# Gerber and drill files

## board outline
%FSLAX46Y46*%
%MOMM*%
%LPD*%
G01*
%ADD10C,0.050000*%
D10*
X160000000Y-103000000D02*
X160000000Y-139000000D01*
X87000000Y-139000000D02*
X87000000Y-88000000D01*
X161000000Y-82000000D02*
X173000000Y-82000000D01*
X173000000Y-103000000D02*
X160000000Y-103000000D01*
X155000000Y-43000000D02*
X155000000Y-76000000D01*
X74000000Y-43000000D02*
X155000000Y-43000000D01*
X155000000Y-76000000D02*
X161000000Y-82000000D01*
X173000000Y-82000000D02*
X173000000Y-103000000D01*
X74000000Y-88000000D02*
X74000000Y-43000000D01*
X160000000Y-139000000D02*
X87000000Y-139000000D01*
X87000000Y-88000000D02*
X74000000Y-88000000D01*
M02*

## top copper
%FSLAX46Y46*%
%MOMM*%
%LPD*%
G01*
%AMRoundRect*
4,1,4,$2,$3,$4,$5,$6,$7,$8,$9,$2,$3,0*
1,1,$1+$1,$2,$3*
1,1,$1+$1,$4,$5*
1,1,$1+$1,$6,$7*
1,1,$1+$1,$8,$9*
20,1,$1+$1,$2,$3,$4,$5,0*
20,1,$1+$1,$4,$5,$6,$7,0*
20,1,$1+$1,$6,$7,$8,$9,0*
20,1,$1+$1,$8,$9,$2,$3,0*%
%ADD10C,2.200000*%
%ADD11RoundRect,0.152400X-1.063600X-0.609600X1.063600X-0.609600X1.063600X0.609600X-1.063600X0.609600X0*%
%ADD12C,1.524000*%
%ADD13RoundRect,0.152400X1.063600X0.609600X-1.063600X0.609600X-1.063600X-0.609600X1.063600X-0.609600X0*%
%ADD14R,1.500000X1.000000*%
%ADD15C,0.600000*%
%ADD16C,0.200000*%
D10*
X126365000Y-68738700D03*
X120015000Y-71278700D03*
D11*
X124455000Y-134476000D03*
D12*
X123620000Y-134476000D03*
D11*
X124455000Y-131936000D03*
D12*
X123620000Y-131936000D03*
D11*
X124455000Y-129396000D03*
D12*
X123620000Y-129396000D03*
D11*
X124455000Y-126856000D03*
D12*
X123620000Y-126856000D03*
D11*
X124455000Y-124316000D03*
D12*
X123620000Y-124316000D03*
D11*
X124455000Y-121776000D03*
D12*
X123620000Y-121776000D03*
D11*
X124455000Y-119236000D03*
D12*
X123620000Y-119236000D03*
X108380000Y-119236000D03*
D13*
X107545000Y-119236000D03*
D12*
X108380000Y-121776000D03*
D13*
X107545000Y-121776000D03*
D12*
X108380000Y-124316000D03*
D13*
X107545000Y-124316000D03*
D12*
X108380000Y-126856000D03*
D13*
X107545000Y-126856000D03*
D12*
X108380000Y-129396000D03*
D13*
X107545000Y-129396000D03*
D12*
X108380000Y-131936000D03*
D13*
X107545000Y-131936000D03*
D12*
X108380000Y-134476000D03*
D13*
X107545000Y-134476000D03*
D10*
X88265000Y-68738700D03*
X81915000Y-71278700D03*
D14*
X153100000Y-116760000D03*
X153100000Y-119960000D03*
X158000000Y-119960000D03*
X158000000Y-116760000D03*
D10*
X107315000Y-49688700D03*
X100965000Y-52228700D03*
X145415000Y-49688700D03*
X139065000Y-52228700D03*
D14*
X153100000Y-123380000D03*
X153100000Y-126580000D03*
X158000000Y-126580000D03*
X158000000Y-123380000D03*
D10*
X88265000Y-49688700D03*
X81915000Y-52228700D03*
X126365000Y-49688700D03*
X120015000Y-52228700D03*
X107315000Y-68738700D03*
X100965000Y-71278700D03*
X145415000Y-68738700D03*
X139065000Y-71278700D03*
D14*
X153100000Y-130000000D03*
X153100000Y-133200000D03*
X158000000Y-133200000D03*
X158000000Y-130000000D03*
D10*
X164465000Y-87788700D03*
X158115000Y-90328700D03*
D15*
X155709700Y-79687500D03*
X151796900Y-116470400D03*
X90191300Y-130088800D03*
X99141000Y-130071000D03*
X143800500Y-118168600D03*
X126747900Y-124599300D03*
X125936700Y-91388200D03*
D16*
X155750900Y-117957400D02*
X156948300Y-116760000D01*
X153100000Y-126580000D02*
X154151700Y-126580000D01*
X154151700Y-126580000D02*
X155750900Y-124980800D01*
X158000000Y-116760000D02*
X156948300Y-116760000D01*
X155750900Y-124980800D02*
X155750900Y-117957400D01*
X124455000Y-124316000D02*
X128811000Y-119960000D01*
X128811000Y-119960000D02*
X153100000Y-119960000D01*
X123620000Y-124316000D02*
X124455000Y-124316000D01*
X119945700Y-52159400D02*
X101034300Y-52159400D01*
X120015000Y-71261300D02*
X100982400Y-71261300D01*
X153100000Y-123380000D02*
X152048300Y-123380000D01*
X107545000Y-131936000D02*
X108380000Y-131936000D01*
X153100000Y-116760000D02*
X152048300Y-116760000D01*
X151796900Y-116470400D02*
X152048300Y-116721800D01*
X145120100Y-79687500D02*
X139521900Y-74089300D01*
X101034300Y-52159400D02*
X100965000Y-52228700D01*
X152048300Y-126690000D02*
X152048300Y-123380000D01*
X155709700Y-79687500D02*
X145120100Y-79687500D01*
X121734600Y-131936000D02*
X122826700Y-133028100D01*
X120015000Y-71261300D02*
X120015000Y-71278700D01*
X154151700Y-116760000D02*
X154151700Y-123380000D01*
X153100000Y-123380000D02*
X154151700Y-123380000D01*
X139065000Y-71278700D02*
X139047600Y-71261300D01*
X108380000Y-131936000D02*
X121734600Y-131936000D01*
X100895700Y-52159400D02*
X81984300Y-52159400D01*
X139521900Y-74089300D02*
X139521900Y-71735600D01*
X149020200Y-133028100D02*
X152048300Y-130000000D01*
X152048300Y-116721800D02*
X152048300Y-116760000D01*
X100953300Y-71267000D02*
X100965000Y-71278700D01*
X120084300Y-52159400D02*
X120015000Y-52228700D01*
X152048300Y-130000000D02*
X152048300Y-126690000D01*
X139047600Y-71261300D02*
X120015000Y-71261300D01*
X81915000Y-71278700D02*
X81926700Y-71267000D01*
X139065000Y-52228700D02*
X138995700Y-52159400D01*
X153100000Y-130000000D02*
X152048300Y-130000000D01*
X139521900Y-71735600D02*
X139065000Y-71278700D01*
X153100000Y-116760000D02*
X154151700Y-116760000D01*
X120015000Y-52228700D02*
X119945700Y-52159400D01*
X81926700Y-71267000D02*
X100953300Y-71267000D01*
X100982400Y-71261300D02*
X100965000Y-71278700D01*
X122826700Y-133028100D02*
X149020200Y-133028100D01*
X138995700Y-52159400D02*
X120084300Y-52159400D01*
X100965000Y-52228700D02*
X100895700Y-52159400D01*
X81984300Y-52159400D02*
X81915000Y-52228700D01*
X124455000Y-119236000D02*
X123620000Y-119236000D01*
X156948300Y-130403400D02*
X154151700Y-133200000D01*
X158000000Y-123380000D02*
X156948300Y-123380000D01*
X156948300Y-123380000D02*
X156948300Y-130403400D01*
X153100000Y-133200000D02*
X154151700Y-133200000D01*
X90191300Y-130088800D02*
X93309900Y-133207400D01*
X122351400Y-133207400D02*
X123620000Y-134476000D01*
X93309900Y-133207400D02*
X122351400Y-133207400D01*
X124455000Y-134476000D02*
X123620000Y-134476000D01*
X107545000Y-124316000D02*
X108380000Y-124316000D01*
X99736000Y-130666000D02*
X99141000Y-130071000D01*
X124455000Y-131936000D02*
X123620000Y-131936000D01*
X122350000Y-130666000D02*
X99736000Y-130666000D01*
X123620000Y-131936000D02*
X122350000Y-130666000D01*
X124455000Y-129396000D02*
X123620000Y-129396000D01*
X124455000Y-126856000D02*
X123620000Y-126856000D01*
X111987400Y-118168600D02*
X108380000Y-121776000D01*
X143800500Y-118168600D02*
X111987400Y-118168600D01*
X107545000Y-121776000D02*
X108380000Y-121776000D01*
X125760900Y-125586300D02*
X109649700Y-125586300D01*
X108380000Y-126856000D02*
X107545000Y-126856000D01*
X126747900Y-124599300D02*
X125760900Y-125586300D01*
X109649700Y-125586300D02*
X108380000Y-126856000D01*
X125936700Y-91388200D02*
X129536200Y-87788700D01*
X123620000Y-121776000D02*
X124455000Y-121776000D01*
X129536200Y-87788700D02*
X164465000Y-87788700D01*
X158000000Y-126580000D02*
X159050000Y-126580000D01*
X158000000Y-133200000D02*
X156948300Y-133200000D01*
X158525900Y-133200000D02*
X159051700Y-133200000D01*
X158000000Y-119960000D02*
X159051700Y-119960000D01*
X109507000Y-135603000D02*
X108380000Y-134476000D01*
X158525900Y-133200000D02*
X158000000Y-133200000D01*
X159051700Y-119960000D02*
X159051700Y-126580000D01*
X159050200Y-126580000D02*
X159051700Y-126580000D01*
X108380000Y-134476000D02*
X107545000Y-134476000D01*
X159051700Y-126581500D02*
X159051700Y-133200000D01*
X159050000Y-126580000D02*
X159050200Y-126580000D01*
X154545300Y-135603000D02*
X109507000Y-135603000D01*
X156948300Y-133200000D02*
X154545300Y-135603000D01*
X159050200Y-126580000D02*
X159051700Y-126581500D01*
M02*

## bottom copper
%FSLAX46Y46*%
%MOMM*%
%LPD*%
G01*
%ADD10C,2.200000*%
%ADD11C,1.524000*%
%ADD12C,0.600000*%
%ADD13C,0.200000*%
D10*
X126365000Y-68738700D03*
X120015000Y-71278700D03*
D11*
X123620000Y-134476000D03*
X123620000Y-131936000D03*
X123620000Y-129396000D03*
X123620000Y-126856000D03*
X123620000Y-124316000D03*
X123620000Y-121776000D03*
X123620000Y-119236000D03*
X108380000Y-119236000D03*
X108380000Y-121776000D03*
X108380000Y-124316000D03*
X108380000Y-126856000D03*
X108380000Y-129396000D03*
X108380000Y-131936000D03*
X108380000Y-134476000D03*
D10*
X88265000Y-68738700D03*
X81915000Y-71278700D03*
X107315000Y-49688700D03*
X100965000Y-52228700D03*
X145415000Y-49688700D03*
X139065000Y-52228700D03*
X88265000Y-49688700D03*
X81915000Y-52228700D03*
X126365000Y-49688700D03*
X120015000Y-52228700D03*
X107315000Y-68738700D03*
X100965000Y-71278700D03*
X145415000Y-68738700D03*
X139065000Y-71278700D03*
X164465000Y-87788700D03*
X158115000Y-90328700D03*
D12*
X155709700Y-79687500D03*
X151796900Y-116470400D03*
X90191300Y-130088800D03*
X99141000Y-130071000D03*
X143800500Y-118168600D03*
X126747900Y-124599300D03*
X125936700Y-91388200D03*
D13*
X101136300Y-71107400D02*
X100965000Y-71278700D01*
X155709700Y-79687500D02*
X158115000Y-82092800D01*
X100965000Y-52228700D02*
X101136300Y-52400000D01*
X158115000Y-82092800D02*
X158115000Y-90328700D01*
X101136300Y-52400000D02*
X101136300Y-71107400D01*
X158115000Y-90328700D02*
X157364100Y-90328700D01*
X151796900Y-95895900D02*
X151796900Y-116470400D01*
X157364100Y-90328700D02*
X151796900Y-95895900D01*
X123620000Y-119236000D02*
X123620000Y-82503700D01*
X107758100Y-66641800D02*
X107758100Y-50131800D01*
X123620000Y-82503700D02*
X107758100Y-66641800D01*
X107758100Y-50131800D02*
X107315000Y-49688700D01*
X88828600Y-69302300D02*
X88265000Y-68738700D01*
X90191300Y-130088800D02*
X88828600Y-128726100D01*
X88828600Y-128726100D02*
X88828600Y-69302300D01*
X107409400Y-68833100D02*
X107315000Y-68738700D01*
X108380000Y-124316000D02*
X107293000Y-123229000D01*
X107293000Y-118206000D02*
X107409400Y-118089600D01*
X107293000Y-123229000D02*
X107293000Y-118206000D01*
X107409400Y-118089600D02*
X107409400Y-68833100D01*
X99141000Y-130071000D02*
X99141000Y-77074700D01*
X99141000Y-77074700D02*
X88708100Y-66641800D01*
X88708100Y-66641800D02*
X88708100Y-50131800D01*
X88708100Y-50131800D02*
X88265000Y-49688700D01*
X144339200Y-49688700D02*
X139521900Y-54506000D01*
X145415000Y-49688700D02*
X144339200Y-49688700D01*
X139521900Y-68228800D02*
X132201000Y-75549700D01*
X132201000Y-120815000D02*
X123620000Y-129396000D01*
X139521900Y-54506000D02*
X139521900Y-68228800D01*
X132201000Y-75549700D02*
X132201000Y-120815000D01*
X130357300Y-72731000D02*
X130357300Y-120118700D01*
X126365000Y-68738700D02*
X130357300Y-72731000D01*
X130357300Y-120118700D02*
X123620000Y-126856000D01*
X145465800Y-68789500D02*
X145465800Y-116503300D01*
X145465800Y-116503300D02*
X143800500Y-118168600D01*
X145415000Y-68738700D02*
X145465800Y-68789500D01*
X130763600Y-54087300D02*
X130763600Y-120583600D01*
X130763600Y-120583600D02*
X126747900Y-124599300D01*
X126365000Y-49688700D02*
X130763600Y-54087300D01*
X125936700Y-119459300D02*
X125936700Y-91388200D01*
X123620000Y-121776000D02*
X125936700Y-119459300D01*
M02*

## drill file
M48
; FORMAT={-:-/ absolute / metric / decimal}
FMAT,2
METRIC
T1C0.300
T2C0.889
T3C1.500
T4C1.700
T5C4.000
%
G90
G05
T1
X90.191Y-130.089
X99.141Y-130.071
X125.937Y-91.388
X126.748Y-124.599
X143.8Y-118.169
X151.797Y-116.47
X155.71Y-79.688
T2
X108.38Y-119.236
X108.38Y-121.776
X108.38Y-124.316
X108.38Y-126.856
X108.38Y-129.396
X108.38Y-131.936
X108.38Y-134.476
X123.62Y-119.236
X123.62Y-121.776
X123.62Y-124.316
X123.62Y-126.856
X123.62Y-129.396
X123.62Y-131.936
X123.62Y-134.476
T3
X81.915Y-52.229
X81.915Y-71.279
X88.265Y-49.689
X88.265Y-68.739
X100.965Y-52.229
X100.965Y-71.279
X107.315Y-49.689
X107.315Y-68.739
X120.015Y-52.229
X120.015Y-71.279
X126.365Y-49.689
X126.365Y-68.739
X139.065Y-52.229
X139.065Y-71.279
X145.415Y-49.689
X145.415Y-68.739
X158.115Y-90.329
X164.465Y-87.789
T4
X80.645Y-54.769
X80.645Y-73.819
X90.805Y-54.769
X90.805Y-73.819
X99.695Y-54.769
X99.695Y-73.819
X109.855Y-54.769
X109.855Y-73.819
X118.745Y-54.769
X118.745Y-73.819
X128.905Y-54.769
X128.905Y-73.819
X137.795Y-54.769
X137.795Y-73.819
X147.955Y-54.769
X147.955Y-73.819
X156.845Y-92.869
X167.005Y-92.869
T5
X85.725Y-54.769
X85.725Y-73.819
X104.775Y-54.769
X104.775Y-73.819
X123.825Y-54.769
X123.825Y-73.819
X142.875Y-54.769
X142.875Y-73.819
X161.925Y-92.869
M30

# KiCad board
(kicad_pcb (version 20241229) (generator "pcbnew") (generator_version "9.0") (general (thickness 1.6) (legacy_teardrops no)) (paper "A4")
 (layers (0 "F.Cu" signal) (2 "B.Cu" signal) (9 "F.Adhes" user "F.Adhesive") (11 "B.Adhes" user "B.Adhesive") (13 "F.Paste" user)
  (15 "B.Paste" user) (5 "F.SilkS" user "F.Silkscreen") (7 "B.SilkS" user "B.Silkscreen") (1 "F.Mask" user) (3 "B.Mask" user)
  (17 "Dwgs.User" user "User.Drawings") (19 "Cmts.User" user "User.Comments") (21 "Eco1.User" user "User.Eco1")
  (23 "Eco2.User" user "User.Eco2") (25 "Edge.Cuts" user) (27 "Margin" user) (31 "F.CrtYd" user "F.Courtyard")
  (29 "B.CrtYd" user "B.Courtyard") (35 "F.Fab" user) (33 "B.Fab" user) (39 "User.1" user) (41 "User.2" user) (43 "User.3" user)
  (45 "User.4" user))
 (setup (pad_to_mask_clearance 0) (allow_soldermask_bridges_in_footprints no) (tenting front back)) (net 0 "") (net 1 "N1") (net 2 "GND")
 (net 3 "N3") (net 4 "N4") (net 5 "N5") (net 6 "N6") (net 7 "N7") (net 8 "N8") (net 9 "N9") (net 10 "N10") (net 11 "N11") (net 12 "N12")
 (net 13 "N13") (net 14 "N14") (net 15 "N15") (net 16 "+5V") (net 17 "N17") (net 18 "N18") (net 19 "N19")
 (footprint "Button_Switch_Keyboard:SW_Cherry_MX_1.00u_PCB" (layer "F.Cu") (at 126.365 68.7387)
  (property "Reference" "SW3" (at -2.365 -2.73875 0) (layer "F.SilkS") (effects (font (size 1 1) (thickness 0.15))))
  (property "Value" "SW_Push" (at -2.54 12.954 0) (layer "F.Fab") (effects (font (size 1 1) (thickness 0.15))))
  (pad "" np_thru_hole circle (at -7.62 5.08) (size 1.7 1.7) (drill 1.7) (layers "*.Cu" "*.Mask"))
  (pad "" np_thru_hole circle (at -2.54 5.08) (size 4 4) (drill 4) (layers "*.Cu" "*.Mask"))
  (pad "" np_thru_hole circle (at 2.54 5.08) (size 1.7 1.7) (drill 1.7) (layers "*.Cu" "*.Mask"))
  (pad "1" thru_hole circle (at 0 0) (size 2.2 2.2) (drill 1.5) (layers "*.Cu" "*.Mask") (remove_unused_layers no) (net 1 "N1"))
  (pad "2" thru_hole circle (at -6.35 2.54) (size 2.2 2.2) (drill 1.5) (layers "*.Cu" "*.Mask") (remove_unused_layers no) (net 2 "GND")))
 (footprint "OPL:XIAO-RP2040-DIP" (layer "F.Cu") (at 116 126.856 180)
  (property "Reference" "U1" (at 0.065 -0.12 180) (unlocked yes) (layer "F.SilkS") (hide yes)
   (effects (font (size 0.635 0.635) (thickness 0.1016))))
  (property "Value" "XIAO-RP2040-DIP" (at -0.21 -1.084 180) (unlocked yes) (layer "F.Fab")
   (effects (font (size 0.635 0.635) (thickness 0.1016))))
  (pad "1" smd roundrect (at -8.455 -7.62) (size 2.432 1.524) (layers "F.Cu" "F.Mask") (roundrect_rratio 0.1) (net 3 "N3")
   (thermal_bridge_angle 45))
  (pad "1" thru_hole circle (at -7.62 -7.62) (size 1.524 1.524) (drill 0.889) (layers "*.Cu" "*.Mask") (remove_unused_layers no)
   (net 3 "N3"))
  (pad "2" smd roundrect (at -8.455 -5.08) (size 2.432 1.524) (layers "F.Cu" "F.Mask") (roundrect_rratio 0.1) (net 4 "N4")
   (thermal_bridge_angle 45))
  (pad "2" thru_hole circle (at -7.62 -5.08) (size 1.524 1.524) (drill 0.889) (layers "*.Cu" "*.Mask") (remove_unused_layers no)
   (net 4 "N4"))
  (pad "3" smd roundrect (at -8.455 -2.54) (size 2.432 1.524) (layers "F.Cu" "F.Mask") (roundrect_rratio 0.1) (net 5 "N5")
   (thermal_bridge_angle 45))
  (pad "3" thru_hole circle (at -7.62 -2.54) (size 1.524 1.524) (drill 0.889) (layers "*.Cu" "*.Mask") (remove_unused_layers no)
   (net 5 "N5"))
  (pad "4" smd roundrect (at -8.455 0) (size 2.432 1.524) (layers "F.Cu" "F.Mask") (roundrect_rratio 0.1) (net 1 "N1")
   (thermal_bridge_angle 45))
  (pad "4" thru_hole circle (at -7.62 0) (size 1.524 1.524) (drill 0.889) (layers "*.Cu" "*.Mask") (remove_unused_layers no) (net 1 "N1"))
  (pad "5" smd roundrect (at -8.455 2.54) (size 2.432 1.524) (layers "F.Cu" "F.Mask") (roundrect_rratio 0.1) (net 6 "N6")
   (thermal_bridge_angle 45))
  (pad "5" thru_hole circle (at -7.62 2.54) (size 1.524 1.524) (drill 0.889) (layers "*.Cu" "*.Mask") (remove_unused_layers no) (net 6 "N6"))
  (pad "6" smd roundrect (at -8.455 5.08) (size 2.432 1.524) (layers "F.Cu" "F.Mask") (roundrect_rratio 0.1) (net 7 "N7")
   (thermal_bridge_angle 45))
  (pad "6" thru_hole circle (at -7.62 5.08) (size 1.524 1.524) (drill 0.889) (layers "*.Cu" "*.Mask") (remove_unused_layers no) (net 7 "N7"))
  (pad "7" smd roundrect (at -8.455 7.62) (size 2.432 1.524) (layers "F.Cu" "F.Mask") (roundrect_rratio 0.1) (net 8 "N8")
   (thermal_bridge_angle 45))
  (pad "7" thru_hole circle (at -7.62 7.62) (size 1.524 1.524) (drill 0.889) (layers "*.Cu" "*.Mask") (remove_unused_layers no) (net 8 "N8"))
  (pad "8" thru_hole circle (at 7.62 7.62 180) (size 1.524 1.524) (drill 0.889) (layers "*.Cu" "*.Mask") (remove_unused_layers no)
   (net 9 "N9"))
  (pad "8" smd roundrect (at 8.455 7.62 180) (size 2.432 1.524) (layers "F.Cu" "F.Mask") (roundrect_rratio 0.1) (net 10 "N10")
   (thermal_bridge_angle 45))
  (pad "9" thru_hole circle (at 7.62 5.08 180) (size 1.524 1.524) (drill 0.889) (layers "*.Cu" "*.Mask") (remove_unused_layers no)
   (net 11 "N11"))
  (pad "9" smd roundrect (at 8.455 5.08 180) (size 2.432 1.524) (layers "F.Cu" "F.Mask") (roundrect_rratio 0.1) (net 11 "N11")
   (thermal_bridge_angle 45))
  (pad "10" thru_hole circle (at 7.62 2.54 180) (size 1.524 1.524) (drill 0.889) (layers "*.Cu" "*.Mask") (remove_unused_layers no)
   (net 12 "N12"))
  (pad "10" smd roundrect (at 8.455 2.54 180) (size 2.432 1.524) (layers "F.Cu" "F.Mask") (roundrect_rratio 0.1) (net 12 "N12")
   (thermal_bridge_angle 45))
  (pad "11" thru_hole circle (at 7.62 0 180) (size 1.524 1.524) (drill 0.889) (layers "*.Cu" "*.Mask") (remove_unused_layers no)
   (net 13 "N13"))
  (pad "11" smd roundrect (at 8.455 0 180) (size 2.432 1.524) (layers "F.Cu" "F.Mask") (roundrect_rratio 0.1) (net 13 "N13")
   (thermal_bridge_angle 45))
  (pad "12" thru_hole circle (at 7.62 -2.54 180) (size 1.524 1.524) (drill 0.889) (layers "*.Cu" "*.Mask") (remove_unused_layers no)
   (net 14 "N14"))
  (pad "12" smd roundrect (at 8.455 -2.54 180) (size 2.432 1.524) (layers "F.Cu" "F.Mask") (roundrect_rratio 0.1) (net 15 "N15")
   (thermal_bridge_angle 45))
  (pad "13" thru_hole circle (at 7.62 -5.08 180) (size 1.524 1.524) (drill 0.889) (layers "*.Cu" "*.Mask") (remove_unused_layers no)
   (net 2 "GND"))
  (pad "13" smd roundrect (at 8.455 -5.08 180) (size 2.432 1.524) (layers "F.Cu" "F.Mask") (roundrect_rratio 0.1) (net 2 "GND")
   (thermal_bridge_angle 45))
  (pad "14" thru_hole circle (at 7.62 -7.62 180) (size 1.524 1.524) (drill 0.889) (layers "*.Cu" "*.Mask") (remove_unused_layers no)
   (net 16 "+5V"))
  (pad "14" smd roundrect (at 8.455 -7.62 180) (size 2.432 1.524) (layers "F.Cu" "F.Mask") (roundrect_rratio 0.1) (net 16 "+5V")
   (thermal_bridge_angle 45)))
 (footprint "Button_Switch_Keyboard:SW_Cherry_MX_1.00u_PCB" (layer "F.Cu") (at 88.265 68.7387)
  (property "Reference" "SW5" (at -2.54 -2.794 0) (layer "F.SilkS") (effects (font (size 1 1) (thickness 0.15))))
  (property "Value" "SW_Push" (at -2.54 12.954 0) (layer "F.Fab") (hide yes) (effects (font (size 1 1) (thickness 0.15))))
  (pad "" np_thru_hole circle (at -7.62 5.08) (size 1.7 1.7) (drill 1.7) (layers "*.Cu" "*.Mask"))
  (pad "" np_thru_hole circle (at -2.54 5.08) (size 4 4) (drill 4) (layers "*.Cu" "*.Mask"))
  (pad "" np_thru_hole circle (at 2.54 5.08) (size 1.7 1.7) (drill 1.7) (layers "*.Cu" "*.Mask"))
  (pad "1" thru_hole circle (at 0 0) (size 2.2 2.2) (drill 1.5) (layers "*.Cu" "*.Mask") (remove_unused_layers no) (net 3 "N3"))
  (pad "2" thru_hole circle (at -6.35 2.54) (size 2.2 2.2) (drill 1.5) (layers "*.Cu" "*.Mask") (remove_unused_layers no) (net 2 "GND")))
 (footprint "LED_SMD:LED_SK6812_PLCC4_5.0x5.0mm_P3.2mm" (layer "F.Cu") (at 155.55 118.36)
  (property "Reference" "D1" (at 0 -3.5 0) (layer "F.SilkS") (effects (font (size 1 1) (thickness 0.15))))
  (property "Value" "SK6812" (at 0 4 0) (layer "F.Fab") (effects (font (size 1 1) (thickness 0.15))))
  (pad "1" smd rect (at -2.45 -1.6 180) (size 1.5 1) (layers "F.Cu" "F.Mask" "F.Paste") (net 2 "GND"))
  (pad "2" smd rect (at -2.45 1.6 180) (size 1.5 1) (layers "F.Cu" "F.Mask" "F.Paste") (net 6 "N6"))
  (pad "3" smd rect (at 2.45 1.6 180) (size 1.5 1) (layers "F.Cu" "F.Mask" "F.Paste") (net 16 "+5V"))
  (pad "4" smd rect (at 2.45 -1.6 180) (size 1.5 1) (layers "F.Cu" "F.Mask" "F.Paste") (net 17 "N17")))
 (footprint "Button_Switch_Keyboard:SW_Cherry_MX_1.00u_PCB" (layer "F.Cu") (at 107.315 49.6887)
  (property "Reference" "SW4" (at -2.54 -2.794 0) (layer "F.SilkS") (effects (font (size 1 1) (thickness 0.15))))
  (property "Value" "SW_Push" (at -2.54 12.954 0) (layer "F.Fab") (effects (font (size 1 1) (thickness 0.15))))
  (pad "" np_thru_hole circle (at -7.62 5.08) (size 1.7 1.7) (drill 1.7) (layers "*.Cu" "*.Mask"))
  (pad "" np_thru_hole circle (at -2.54 5.08) (size 4 4) (drill 4) (layers "*.Cu" "*.Mask"))
  (pad "" np_thru_hole circle (at 2.54 5.08) (size 1.7 1.7) (drill 1.7) (layers "*.Cu" "*.Mask"))
  (pad "1" thru_hole circle (at 0 0) (size 2.2 2.2) (drill 1.5) (layers "*.Cu" "*.Mask") (remove_unused_layers no) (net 8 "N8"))
  (pad "2" thru_hole circle (at -6.35 2.54) (size 2.2 2.2) (drill 1.5) (layers "*.Cu" "*.Mask") (remove_unused_layers no) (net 2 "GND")))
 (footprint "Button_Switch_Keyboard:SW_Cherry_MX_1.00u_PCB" (layer "F.Cu") (at 145.415 49.6887)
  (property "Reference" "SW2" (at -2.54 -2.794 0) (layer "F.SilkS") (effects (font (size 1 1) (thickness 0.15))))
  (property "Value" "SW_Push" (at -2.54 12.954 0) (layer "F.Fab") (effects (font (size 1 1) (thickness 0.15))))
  (pad "" np_thru_hole circle (at -7.62 5.08) (size 1.7 1.7) (drill 1.7) (layers "*.Cu" "*.Mask"))
  (pad "" np_thru_hole circle (at -2.54 5.08) (size 4 4) (drill 4) (layers "*.Cu" "*.Mask"))
  (pad "" np_thru_hole circle (at 2.54 5.08) (size 1.7 1.7) (drill 1.7) (layers "*.Cu" "*.Mask"))
  (pad "1" thru_hole circle (at 0 0) (size 2.2 2.2) (drill 1.5) (layers "*.Cu" "*.Mask") (remove_unused_layers no) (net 5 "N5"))
  (pad "2" thru_hole circle (at -6.35 2.54) (size 2.2 2.2) (drill 1.5) (layers "*.Cu" "*.Mask") (remove_unused_layers no) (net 2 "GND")))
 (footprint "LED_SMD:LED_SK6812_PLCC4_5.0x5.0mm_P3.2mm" (layer "F.Cu") (at 155.55 124.98)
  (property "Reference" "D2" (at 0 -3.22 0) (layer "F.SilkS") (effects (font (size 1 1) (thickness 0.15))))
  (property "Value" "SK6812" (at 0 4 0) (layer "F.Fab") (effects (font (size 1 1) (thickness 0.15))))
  (pad "1" smd rect (at -2.45 -1.6 180) (size 1.5 1) (layers "F.Cu" "F.Mask" "F.Paste") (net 2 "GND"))
  (pad "2" smd rect (at -2.45 1.6 180) (size 1.5 1) (layers "F.Cu" "F.Mask" "F.Paste") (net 17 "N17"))
  (pad "3" smd rect (at 2.45 1.6 180) (size 1.5 1) (layers "F.Cu" "F.Mask" "F.Paste") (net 16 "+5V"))
  (pad "4" smd rect (at 2.45 -1.6 180) (size 1.5 1) (layers "F.Cu" "F.Mask" "F.Paste") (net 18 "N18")))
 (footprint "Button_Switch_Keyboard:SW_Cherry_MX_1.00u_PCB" (layer "F.Cu") (at 88.265 49.6887)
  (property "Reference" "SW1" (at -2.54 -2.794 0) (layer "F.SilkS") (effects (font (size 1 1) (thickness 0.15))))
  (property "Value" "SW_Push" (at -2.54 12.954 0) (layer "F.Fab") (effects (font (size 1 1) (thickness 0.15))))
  (pad "" np_thru_hole circle (at -7.62 5.08) (size 1.7 1.7) (drill 1.7) (layers "*.Cu" "*.Mask"))
  (pad "" np_thru_hole circle (at -2.54 5.08) (size 4 4) (drill 4) (layers "*.Cu" "*.Mask"))
  (pad "" np_thru_hole circle (at 2.54 5.08) (size 1.7 1.7) (drill 1.7) (layers "*.Cu" "*.Mask"))
  (pad "1" thru_hole circle (at 0 0) (size 2.2 2.2) (drill 1.5) (layers "*.Cu" "*.Mask") (remove_unused_layers no) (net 4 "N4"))
  (pad "2" thru_hole circle (at -6.35 2.54) (size 2.2 2.2) (drill 1.5) (layers "*.Cu" "*.Mask") (remove_unused_layers no) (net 2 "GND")))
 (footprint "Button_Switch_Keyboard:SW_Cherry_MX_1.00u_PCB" (layer "F.Cu") (at 126.365 49.6887)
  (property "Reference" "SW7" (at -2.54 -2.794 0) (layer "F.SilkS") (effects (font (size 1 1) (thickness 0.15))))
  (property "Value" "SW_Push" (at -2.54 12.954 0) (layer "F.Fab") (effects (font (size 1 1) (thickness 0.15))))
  (pad "" np_thru_hole circle (at -7.62 5.08) (size 1.7 1.7) (drill 1.7) (layers "*.Cu" "*.Mask"))
  (pad "" np_thru_hole circle (at -2.54 5.08) (size 4 4) (drill 4) (layers "*.Cu" "*.Mask"))
  (pad "" np_thru_hole circle (at 2.54 5.08) (size 1.7 1.7) (drill 1.7) (layers "*.Cu" "*.Mask"))
  (pad "1" thru_hole circle (at 0 0) (size 2.2 2.2) (drill 1.5) (layers "*.Cu" "*.Mask") (remove_unused_layers no) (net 13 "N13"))
  (pad "2" thru_hole circle (at -6.35 2.54) (size 2.2 2.2) (drill 1.5) (layers "*.Cu" "*.Mask") (remove_unused_layers no) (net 2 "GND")))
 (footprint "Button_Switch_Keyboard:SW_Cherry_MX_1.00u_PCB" (layer "F.Cu") (at 107.315 68.7387)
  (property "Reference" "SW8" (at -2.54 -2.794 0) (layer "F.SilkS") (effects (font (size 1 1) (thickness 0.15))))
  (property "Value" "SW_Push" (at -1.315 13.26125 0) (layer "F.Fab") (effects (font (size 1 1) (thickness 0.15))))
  (pad "" np_thru_hole circle (at -7.62 5.08) (size 1.7 1.7) (drill 1.7) (layers "*.Cu" "*.Mask"))
  (pad "" np_thru_hole circle (at -2.54 5.08) (size 4 4) (drill 4) (layers "*.Cu" "*.Mask"))
  (pad "" np_thru_hole circle (at 2.54 5.08) (size 1.7 1.7) (drill 1.7) (layers "*.Cu" "*.Mask"))
  (pad "1" thru_hole circle (at 0 0) (size 2.2 2.2) (drill 1.5) (layers "*.Cu" "*.Mask") (remove_unused_layers no) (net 12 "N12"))
  (pad "2" thru_hole circle (at -6.35 2.54) (size 2.2 2.2) (drill 1.5) (layers "*.Cu" "*.Mask") (remove_unused_layers no) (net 2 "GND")))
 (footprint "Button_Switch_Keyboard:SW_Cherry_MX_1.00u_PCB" (layer "F.Cu") (at 145.415 68.7387)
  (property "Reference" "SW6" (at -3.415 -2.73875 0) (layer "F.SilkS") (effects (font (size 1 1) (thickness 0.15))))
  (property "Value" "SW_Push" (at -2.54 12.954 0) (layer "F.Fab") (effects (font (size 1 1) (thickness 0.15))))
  (pad "" np_thru_hole circle (at -7.62 5.08) (size 1.7 1.7) (drill 1.7) (layers "*.Cu" "*.Mask"))
  (pad "" np_thru_hole circle (at -2.54 5.08) (size 4 4) (drill 4) (layers "*.Cu" "*.Mask"))
  (pad "" np_thru_hole circle (at 2.54 5.08) (size 1.7 1.7) (drill 1.7) (layers "*.Cu" "*.Mask"))
  (pad "1" thru_hole circle (at 0 0) (size 2.2 2.2) (drill 1.5) (layers "*.Cu" "*.Mask") (remove_unused_layers no) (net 11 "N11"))
  (pad "2" thru_hole circle (at -6.35 2.54) (size 2.2 2.2) (drill 1.5) (layers "*.Cu" "*.Mask") (remove_unused_layers no) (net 2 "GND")))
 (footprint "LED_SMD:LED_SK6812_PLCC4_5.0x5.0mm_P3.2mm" (layer "F.Cu") (at 155.55 131.6)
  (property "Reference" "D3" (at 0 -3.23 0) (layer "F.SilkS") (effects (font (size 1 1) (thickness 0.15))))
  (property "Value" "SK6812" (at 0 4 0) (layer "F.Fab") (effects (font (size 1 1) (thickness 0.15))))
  (pad "1" smd rect (at -2.45 -1.6 180) (size 1.5 1) (layers "F.Cu" "F.Mask" "F.Paste") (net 2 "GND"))
  (pad "2" smd rect (at -2.45 1.6 180) (size 1.5 1) (layers "F.Cu" "F.Mask" "F.Paste") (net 18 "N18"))
  (pad "3" smd rect (at 2.45 1.6 180) (size 1.5 1) (layers "F.Cu" "F.Mask" "F.Paste") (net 16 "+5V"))
  (pad "4" smd rect (at 2.45 -1.6 180) (size 1.5 1) (layers "F.Cu" "F.Mask" "F.Paste") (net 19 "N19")))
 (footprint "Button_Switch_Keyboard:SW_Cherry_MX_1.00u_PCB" (layer "F.Cu") (at 164.465 87.7887)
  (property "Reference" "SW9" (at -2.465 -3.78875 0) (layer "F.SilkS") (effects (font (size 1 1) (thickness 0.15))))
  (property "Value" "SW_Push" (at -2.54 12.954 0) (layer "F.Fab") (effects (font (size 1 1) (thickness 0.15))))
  (pad "" np_thru_hole circle (at -7.62 5.08) (size 1.7 1.7) (drill 1.7) (layers "*.Cu" "*.Mask"))
  (pad "" np_thru_hole circle (at -2.54 5.08) (size 4 4) (drill 4) (layers "*.Cu" "*.Mask"))
  (pad "" np_thru_hole circle (at 2.54 5.08) (size 1.7 1.7) (drill 1.7) (layers "*.Cu" "*.Mask"))
  (pad "1" thru_hole circle (at 0 0) (size 2.2 2.2) (drill 1.5) (layers "*.Cu" "*.Mask") (remove_unused_layers no) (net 7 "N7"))
  (pad "2" thru_hole circle (at -6.35 2.54) (size 2.2 2.2) (drill 1.5) (layers "*.Cu" "*.Mask") (remove_unused_layers no) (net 2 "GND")))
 (gr_line (start 160 103) (end 160 139) (stroke (width 0.05) (type default)) (layer "Edge.Cuts"))
 (gr_line (start 87 139) (end 87 88) (stroke (width 0.05) (type default)) (layer "Edge.Cuts"))
 (gr_line (start 161 82) (end 173 82) (stroke (width 0.05) (type default)) (layer "Edge.Cuts"))
 (gr_line (start 173 103) (end 160 103) (stroke (width 0.05) (type default)) (layer "Edge.Cuts"))
 (gr_line (start 155 43) (end 155 76) (stroke (width 0.05) (type default)) (layer "Edge.Cuts"))
 (gr_line (start 74 43) (end 155 43) (stroke (width 0.05) (type default)) (layer "Edge.Cuts"))
 (gr_line (start 155 76) (end 161 82) (stroke (width 0.05) (type default)) (layer "Edge.Cuts"))
 (gr_line (start 173 82) (end 173 103) (stroke (width 0.05) (type default)) (layer "Edge.Cuts"))
 (gr_line (start 74 88) (end 74 43) (stroke (width 0.05) (type default)) (layer "Edge.Cuts"))
 (gr_line (start 160 139) (end 87 139) (stroke (width 0.05) (type default)) (layer "Edge.Cuts"))
 (gr_line (start 87 88) (end 74 88) (stroke (width 0.05) (type default)) (layer "Edge.Cuts"))
 (segment (start 155.7509 117.9574) (end 156.9483 116.76) (width 0.2) (layer "F.Cu") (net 17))
 (segment (start 153.1 126.58) (end 154.1517 126.58) (width 0.2) (layer "F.Cu") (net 17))
 (segment (start 154.1517 126.58) (end 155.7509 124.9808) (width 0.2) (layer "F.Cu") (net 17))
 (segment (start 158 116.76) (end 156.9483 116.76) (width 0.2) (layer "F.Cu") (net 17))
 (segment (start 155.7509 124.9808) (end 155.7509 117.9574) (width 0.2) (layer "F.Cu") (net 17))
 (segment (start 124.455 124.316) (end 128.811 119.96) (width 0.2) (layer "F.Cu") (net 6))
 (segment (start 128.811 119.96) (end 153.1 119.96) (width 0.2) (layer "F.Cu") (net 6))
 (segment (start 123.62 124.316) (end 124.455 124.316) (width 0.2) (layer "F.Cu") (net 6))
 (segment (start 119.9457 52.1594) (end 101.0343 52.1594) (width 0.2) (layer "F.Cu") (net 2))
 (segment (start 120.015 71.2613) (end 100.9824 71.2613) (width 0.2) (layer "F.Cu") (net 2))
 (segment (start 153.1 123.38) (end 152.0483 123.38) (width 0.2) (layer "F.Cu") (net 2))
 (segment (start 107.545 131.936) (end 108.38 131.936) (width 0.2) (layer "F.Cu") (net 2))
 (segment (start 153.1 116.76) (end 152.0483 116.76) (width 0.2) (layer "F.Cu") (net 2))
 (segment (start 151.7969 116.4704) (end 152.0483 116.7218) (width 0.2) (layer "F.Cu") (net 2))
 (segment (start 145.1201 79.6875) (end 139.5219 74.0893) (width 0.2) (layer "F.Cu") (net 2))
 (segment (start 101.0343 52.1594) (end 100.965 52.2287) (width 0.2) (layer "F.Cu") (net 2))
 (segment (start 152.0483 126.69) (end 152.0483 123.38) (width 0.2) (layer "F.Cu") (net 2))
 (segment (start 155.7097 79.6875) (end 145.1201 79.6875) (width 0.2) (layer "F.Cu") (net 2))
 (segment (start 121.7346 131.936) (end 122.8267 133.0281) (width 0.2) (layer "F.Cu") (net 2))
 (segment (start 120.015 71.2613) (end 120.015 71.2787) (width 0.2) (layer "F.Cu") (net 2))
 (segment (start 154.1517 116.76) (end 154.1517 123.38) (width 0.2) (layer "F.Cu") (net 2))
 (segment (start 153.1 123.38) (end 154.1517 123.38) (width 0.2) (layer "F.Cu") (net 2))
 (segment (start 139.065 71.2787) (end 139.0476 71.2613) (width 0.2) (layer "F.Cu") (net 2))
 (segment (start 108.38 131.936) (end 121.7346 131.936) (width 0.2) (layer "F.Cu") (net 2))
 (segment (start 100.8957 52.1594) (end 81.9843 52.1594) (width 0.2) (layer "F.Cu") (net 2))
 (segment (start 139.5219 74.0893) (end 139.5219 71.7356) (width 0.2) (layer "F.Cu") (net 2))
 (segment (start 149.0202 133.0281) (end 152.0483 130) (width 0.2) (layer "F.Cu") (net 2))
 (segment (start 152.0483 116.7218) (end 152.0483 116.76) (width 0.2) (layer "F.Cu") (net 2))
 (segment (start 100.9533 71.267) (end 100.965 71.2787) (width 0.2) (layer "F.Cu") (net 2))
 (segment (start 120.0843 52.1594) (end 120.015 52.2287) (width 0.2) (layer "F.Cu") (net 2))
 (segment (start 152.0483 130) (end 152.0483 126.69) (width 0.2) (layer "F.Cu") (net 2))
 (segment (start 139.0476 71.2613) (end 120.015 71.2613) (width 0.2) (layer "F.Cu") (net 2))
 (segment (start 81.915 71.2787) (end 81.9267 71.267) (width 0.2) (layer "F.Cu") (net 2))
 (segment (start 139.065 52.2287) (end 138.9957 52.1594) (width 0.2) (layer "F.Cu") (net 2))
 (segment (start 153.1 130) (end 152.0483 130) (width 0.2) (layer "F.Cu") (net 2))
 (segment (start 139.5219 71.7356) (end 139.065 71.2787) (width 0.2) (layer "F.Cu") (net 2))
 (segment (start 153.1 116.76) (end 154.1517 116.76) (width 0.2) (layer "F.Cu") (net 2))
 (segment (start 120.015 52.2287) (end 119.9457 52.1594) (width 0.2) (layer "F.Cu") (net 2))
 (segment (start 81.9267 71.267) (end 100.9533 71.267) (width 0.2) (layer "F.Cu") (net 2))
 (segment (start 100.9824 71.2613) (end 100.965 71.2787) (width 0.2) (layer "F.Cu") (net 2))
 (segment (start 122.8267 133.0281) (end 149.0202 133.0281) (width 0.2) (layer "F.Cu") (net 2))
 (segment (start 138.9957 52.1594) (end 120.0843 52.1594) (width 0.2) (layer "F.Cu") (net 2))
 (segment (start 100.965 52.2287) (end 100.8957 52.1594) (width 0.2) (layer "F.Cu") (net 2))
 (segment (start 81.9843 52.1594) (end 81.915 52.2287) (width 0.2) (layer "F.Cu") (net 2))
 (via (at 155.7097 79.6875) (size 0.6) (drill 0.3) (layers "F.Cu" "B.Cu") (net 2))
 (via (at 151.7969 116.4704) (size 0.6) (drill 0.3) (layers "F.Cu" "B.Cu") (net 2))
 (segment (start 101.1363 71.1074) (end 100.965 71.2787) (width 0.2) (layer "B.Cu") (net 2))
 (segment (start 155.7097 79.6875) (end 158.115 82.0928) (width 0.2) (layer "B.Cu") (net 2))
 (segment (start 100.965 52.2287) (end 101.1363 52.4) (width 0.2) (layer "B.Cu") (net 2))
 (segment (start 158.115 82.0928) (end 158.115 90.3287) (width 0.2) (layer "B.Cu") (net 2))
 (segment (start 101.1363 52.4) (end 101.1363 71.1074) (width 0.2) (layer "B.Cu") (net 2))
 (segment (start 158.115 90.3287) (end 157.3641 90.3287) (width 0.2) (layer "B.Cu") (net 2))
 (segment (start 151.7969 95.8959) (end 151.7969 116.4704) (width 0.2) (layer "B.Cu") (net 2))
 (segment (start 157.3641 90.3287) (end 151.7969 95.8959) (width 0.2) (layer "B.Cu") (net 2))
 (segment (start 124.455 119.236) (end 123.62 119.236) (width 0.2) (layer "F.Cu") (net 8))
 (segment (start 123.62 119.236) (end 123.62 82.5037) (width 0.2) (layer "B.Cu") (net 8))
 (segment (start 107.7581 66.6418) (end 107.7581 50.1318) (width 0.2) (layer "B.Cu") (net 8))
 (segment (start 123.62 82.5037) (end 107.7581 66.6418) (width 0.2) (layer "B.Cu") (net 8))
 (segment (start 107.7581 50.1318) (end 107.315 49.6887) (width 0.2) (layer "B.Cu") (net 8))
 (segment (start 156.9483 130.4034) (end 154.1517 133.2) (width 0.2) (layer "F.Cu") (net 18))
 (segment (start 158 123.38) (end 156.9483 123.38) (width 0.2) (layer "F.Cu") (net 18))
 (segment (start 156.9483 123.38) (end 156.9483 130.4034) (width 0.2) (layer "F.Cu") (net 18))
 (segment (start 153.1 133.2) (end 154.1517 133.2) (width 0.2) (layer "F.Cu") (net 18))
 (segment (start 90.1913 130.0888) (end 93.3099 133.2074) (width 0.2) (layer "F.Cu") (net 3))
 (segment (start 122.3514 133.2074) (end 123.62 134.476) (width 0.2) (layer "F.Cu") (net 3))
 (segment (start 93.3099 133.2074) (end 122.3514 133.2074) (width 0.2) (layer "F.Cu") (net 3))
 (segment (start 124.455 134.476) (end 123.62 134.476) (width 0.2) (layer "F.Cu") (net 3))
 (via (at 90.1913 130.0888) (size 0.6) (drill 0.3) (layers "F.Cu" "B.Cu") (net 3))
 (segment (start 88.8286 69.3023) (end 88.265 68.7387) (width 0.2) (layer "B.Cu") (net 3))
 (segment (start 90.1913 130.0888) (end 88.8286 128.7261) (width 0.2) (layer "B.Cu") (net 3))
 (segment (start 88.8286 128.7261) (end 88.8286 69.3023) (width 0.2) (layer "B.Cu") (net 3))
 (segment (start 107.545 124.316) (end 108.38 124.316) (width 0.2) (layer "F.Cu") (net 12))
 (segment (start 107.4094 68.8331) (end 107.315 68.7387) (width 0.2) (layer "B.Cu") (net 12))
 (segment (start 108.38 124.316) (end 107.293 123.229) (width 0.2) (layer "B.Cu") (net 12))
 (segment (start 107.293 118.206) (end 107.4094 118.0896) (width 0.2) (layer "B.Cu") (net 12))
 (segment (start 107.293 123.229) (end 107.293 118.206) (width 0.2) (layer "B.Cu") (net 12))
 (segment (start 107.4094 118.0896) (end 107.4094 68.8331) (width 0.2) (layer "B.Cu") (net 12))
 (segment (start 99.736 130.666) (end 99.141 130.071) (width 0.2) (layer "F.Cu") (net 4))
 (segment (start 124.455 131.936) (end 123.62 131.936) (width 0.2) (layer "F.Cu") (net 4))
 (segment (start 122.35 130.666) (end 99.736 130.666) (width 0.2) (layer "F.Cu") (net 4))
 (segment (start 123.62 131.936) (end 122.35 130.666) (width 0.2) (layer "F.Cu") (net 4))
 (via (at 99.141 130.071) (size 0.6) (drill 0.3) (layers "F.Cu" "B.Cu") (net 4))
 (segment (start 99.141 130.071) (end 99.141 77.0747) (width 0.2) (layer "B.Cu") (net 4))
 (segment (start 99.141 77.0747) (end 88.7081 66.6418) (width 0.2) (layer "B.Cu") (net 4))
 (segment (start 88.7081 66.6418) (end 88.7081 50.1318) (width 0.2) (layer "B.Cu") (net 4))
 (segment (start 88.7081 50.1318) (end 88.265 49.6887) (width 0.2) (layer "B.Cu") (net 4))
 (segment (start 124.455 129.396) (end 123.62 129.396) (width 0.2) (layer "F.Cu") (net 5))
 (segment (start 144.3392 49.6887) (end 139.5219 54.506) (width 0.2) (layer "B.Cu") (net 5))
 (segment (start 145.415 49.6887) (end 144.3392 49.6887) (width 0.2) (layer "B.Cu") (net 5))
 (segment (start 139.5219 68.2288) (end 132.201 75.5497) (width 0.2) (layer "B.Cu") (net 5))
 (segment (start 132.201 120.815) (end 123.62 129.396) (width 0.2) (layer "B.Cu") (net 5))
 (segment (start 139.5219 54.506) (end 139.5219 68.2288) (width 0.2) (layer "B.Cu") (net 5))
 (segment (start 132.201 75.5497) (end 132.201 120.815) (width 0.2) (layer "B.Cu") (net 5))
 (segment (start 124.455 126.856) (end 123.62 126.856) (width 0.2) (layer "F.Cu") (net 1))
 (segment (start 130.3573 72.731) (end 130.3573 120.1187) (width 0.2) (layer "B.Cu") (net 1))
 (segment (start 126.365 68.7387) (end 130.3573 72.731) (width 0.2) (layer "B.Cu") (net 1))
 (segment (start 130.3573 120.1187) (end 123.62 126.856) (width 0.2) (layer "B.Cu") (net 1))
 (segment (start 111.9874 118.1686) (end 108.38 121.776) (width 0.2) (layer "F.Cu") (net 11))
 (segment (start 143.8005 118.1686) (end 111.9874 118.1686) (width 0.2) (layer "F.Cu") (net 11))
 (segment (start 107.545 121.776) (end 108.38 121.776) (width 0.2) (layer "F.Cu") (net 11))
 (via (at 143.8005 118.1686) (size 0.6) (drill 0.3) (layers "F.Cu" "B.Cu") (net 11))
 (segment (start 145.4658 68.7895) (end 145.4658 116.5033) (width 0.2) (layer "B.Cu") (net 11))
 (segment (start 145.4658 116.5033) (end 143.8005 118.1686) (width 0.2) (layer "B.Cu") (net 11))
 (segment (start 145.415 68.7387) (end 145.4658 68.7895) (width 0.2) (layer "B.Cu") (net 11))
 (segment (start 125.7609 125.5863) (end 109.6497 125.5863) (width 0.2) (layer "F.Cu") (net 13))
 (segment (start 108.38 126.856) (end 107.545 126.856) (width 0.2) (layer "F.Cu") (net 13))
 (segment (start 126.7479 124.5993) (end 125.7609 125.5863) (width 0.2) (layer "F.Cu") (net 13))
 (segment (start 109.6497 125.5863) (end 108.38 126.856) (width 0.2) (layer "F.Cu") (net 13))
 (via (at 126.7479 124.5993) (size 0.6) (drill 0.3) (layers "F.Cu" "B.Cu") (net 13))
 (segment (start 130.7636 54.0873) (end 130.7636 120.5836) (width 0.2) (layer "B.Cu") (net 13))
 (segment (start 130.7636 120.5836) (end 126.7479 124.5993) (width 0.2) (layer "B.Cu") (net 13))
 (segment (start 126.365 49.6887) (end 130.7636 54.0873) (width 0.2) (layer "B.Cu") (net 13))
 (segment (start 125.9367 91.3882) (end 129.5362 87.7887) (width 0.2) (layer "F.Cu") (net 7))
 (segment (start 123.62 121.776) (end 124.455 121.776) (width 0.2) (layer "F.Cu") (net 7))
 (segment (start 129.5362 87.7887) (end 164.465 87.7887) (width 0.2) (layer "F.Cu") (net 7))
 (via (at 125.9367 91.3882) (size 0.6) (drill 0.3) (layers "F.Cu" "B.Cu") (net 7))
 (segment (start 125.9367 119.4593) (end 125.9367 91.3882) (width 0.2) (layer "B.Cu") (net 7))
 (segment (start 123.62 121.776) (end 125.9367 119.4593) (width 0.2) (layer "B.Cu") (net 7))
 (segment (start 158 126.58) (end 159.05 126.58) (width 0.2) (layer "F.Cu") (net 16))
 (segment (start 158 133.2) (end 156.9483 133.2) (width 0.2) (layer "F.Cu") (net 16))
 (segment (start 158.5259 133.2) (end 159.0517 133.2) (width 0.2) (layer "F.Cu") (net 16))
 (segment (start 158 119.96) (end 159.0517 119.96) (width 0.2) (layer "F.Cu") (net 16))
 (segment (start 109.507 135.603) (end 108.38 134.476) (width 0.2) (layer "F.Cu") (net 16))
 (segment (start 158.5259 133.2) (end 158 133.2) (width 0.2) (layer "F.Cu") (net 16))
 (segment (start 159.0517 119.96) (end 159.0517 126.58) (width 0.2) (layer "F.Cu") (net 16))
 (segment (start 159.0502 126.58) (end 159.0517 126.58) (width 0.2) (layer "F.Cu") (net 16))
 (segment (start 108.38 134.476) (end 107.545 134.476) (width 0.2) (layer "F.Cu") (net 16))
 (segment (start 159.0517 126.5815) (end 159.0517 133.2) (width 0.2) (layer "F.Cu") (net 16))
 (segment (start 159.05 126.58) (end 159.0502 126.58) (width 0.2) (layer "F.Cu") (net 16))
 (segment (start 154.5453 135.603) (end 109.507 135.603) (width 0.2) (layer "F.Cu") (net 16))
 (segment (start 156.9483 133.2) (end 154.5453 135.603) (width 0.2) (layer "F.Cu") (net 16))
 (segment (start 159.0502 126.58) (end 159.0517 126.5815) (width 0.2) (layer "F.Cu") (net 16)))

